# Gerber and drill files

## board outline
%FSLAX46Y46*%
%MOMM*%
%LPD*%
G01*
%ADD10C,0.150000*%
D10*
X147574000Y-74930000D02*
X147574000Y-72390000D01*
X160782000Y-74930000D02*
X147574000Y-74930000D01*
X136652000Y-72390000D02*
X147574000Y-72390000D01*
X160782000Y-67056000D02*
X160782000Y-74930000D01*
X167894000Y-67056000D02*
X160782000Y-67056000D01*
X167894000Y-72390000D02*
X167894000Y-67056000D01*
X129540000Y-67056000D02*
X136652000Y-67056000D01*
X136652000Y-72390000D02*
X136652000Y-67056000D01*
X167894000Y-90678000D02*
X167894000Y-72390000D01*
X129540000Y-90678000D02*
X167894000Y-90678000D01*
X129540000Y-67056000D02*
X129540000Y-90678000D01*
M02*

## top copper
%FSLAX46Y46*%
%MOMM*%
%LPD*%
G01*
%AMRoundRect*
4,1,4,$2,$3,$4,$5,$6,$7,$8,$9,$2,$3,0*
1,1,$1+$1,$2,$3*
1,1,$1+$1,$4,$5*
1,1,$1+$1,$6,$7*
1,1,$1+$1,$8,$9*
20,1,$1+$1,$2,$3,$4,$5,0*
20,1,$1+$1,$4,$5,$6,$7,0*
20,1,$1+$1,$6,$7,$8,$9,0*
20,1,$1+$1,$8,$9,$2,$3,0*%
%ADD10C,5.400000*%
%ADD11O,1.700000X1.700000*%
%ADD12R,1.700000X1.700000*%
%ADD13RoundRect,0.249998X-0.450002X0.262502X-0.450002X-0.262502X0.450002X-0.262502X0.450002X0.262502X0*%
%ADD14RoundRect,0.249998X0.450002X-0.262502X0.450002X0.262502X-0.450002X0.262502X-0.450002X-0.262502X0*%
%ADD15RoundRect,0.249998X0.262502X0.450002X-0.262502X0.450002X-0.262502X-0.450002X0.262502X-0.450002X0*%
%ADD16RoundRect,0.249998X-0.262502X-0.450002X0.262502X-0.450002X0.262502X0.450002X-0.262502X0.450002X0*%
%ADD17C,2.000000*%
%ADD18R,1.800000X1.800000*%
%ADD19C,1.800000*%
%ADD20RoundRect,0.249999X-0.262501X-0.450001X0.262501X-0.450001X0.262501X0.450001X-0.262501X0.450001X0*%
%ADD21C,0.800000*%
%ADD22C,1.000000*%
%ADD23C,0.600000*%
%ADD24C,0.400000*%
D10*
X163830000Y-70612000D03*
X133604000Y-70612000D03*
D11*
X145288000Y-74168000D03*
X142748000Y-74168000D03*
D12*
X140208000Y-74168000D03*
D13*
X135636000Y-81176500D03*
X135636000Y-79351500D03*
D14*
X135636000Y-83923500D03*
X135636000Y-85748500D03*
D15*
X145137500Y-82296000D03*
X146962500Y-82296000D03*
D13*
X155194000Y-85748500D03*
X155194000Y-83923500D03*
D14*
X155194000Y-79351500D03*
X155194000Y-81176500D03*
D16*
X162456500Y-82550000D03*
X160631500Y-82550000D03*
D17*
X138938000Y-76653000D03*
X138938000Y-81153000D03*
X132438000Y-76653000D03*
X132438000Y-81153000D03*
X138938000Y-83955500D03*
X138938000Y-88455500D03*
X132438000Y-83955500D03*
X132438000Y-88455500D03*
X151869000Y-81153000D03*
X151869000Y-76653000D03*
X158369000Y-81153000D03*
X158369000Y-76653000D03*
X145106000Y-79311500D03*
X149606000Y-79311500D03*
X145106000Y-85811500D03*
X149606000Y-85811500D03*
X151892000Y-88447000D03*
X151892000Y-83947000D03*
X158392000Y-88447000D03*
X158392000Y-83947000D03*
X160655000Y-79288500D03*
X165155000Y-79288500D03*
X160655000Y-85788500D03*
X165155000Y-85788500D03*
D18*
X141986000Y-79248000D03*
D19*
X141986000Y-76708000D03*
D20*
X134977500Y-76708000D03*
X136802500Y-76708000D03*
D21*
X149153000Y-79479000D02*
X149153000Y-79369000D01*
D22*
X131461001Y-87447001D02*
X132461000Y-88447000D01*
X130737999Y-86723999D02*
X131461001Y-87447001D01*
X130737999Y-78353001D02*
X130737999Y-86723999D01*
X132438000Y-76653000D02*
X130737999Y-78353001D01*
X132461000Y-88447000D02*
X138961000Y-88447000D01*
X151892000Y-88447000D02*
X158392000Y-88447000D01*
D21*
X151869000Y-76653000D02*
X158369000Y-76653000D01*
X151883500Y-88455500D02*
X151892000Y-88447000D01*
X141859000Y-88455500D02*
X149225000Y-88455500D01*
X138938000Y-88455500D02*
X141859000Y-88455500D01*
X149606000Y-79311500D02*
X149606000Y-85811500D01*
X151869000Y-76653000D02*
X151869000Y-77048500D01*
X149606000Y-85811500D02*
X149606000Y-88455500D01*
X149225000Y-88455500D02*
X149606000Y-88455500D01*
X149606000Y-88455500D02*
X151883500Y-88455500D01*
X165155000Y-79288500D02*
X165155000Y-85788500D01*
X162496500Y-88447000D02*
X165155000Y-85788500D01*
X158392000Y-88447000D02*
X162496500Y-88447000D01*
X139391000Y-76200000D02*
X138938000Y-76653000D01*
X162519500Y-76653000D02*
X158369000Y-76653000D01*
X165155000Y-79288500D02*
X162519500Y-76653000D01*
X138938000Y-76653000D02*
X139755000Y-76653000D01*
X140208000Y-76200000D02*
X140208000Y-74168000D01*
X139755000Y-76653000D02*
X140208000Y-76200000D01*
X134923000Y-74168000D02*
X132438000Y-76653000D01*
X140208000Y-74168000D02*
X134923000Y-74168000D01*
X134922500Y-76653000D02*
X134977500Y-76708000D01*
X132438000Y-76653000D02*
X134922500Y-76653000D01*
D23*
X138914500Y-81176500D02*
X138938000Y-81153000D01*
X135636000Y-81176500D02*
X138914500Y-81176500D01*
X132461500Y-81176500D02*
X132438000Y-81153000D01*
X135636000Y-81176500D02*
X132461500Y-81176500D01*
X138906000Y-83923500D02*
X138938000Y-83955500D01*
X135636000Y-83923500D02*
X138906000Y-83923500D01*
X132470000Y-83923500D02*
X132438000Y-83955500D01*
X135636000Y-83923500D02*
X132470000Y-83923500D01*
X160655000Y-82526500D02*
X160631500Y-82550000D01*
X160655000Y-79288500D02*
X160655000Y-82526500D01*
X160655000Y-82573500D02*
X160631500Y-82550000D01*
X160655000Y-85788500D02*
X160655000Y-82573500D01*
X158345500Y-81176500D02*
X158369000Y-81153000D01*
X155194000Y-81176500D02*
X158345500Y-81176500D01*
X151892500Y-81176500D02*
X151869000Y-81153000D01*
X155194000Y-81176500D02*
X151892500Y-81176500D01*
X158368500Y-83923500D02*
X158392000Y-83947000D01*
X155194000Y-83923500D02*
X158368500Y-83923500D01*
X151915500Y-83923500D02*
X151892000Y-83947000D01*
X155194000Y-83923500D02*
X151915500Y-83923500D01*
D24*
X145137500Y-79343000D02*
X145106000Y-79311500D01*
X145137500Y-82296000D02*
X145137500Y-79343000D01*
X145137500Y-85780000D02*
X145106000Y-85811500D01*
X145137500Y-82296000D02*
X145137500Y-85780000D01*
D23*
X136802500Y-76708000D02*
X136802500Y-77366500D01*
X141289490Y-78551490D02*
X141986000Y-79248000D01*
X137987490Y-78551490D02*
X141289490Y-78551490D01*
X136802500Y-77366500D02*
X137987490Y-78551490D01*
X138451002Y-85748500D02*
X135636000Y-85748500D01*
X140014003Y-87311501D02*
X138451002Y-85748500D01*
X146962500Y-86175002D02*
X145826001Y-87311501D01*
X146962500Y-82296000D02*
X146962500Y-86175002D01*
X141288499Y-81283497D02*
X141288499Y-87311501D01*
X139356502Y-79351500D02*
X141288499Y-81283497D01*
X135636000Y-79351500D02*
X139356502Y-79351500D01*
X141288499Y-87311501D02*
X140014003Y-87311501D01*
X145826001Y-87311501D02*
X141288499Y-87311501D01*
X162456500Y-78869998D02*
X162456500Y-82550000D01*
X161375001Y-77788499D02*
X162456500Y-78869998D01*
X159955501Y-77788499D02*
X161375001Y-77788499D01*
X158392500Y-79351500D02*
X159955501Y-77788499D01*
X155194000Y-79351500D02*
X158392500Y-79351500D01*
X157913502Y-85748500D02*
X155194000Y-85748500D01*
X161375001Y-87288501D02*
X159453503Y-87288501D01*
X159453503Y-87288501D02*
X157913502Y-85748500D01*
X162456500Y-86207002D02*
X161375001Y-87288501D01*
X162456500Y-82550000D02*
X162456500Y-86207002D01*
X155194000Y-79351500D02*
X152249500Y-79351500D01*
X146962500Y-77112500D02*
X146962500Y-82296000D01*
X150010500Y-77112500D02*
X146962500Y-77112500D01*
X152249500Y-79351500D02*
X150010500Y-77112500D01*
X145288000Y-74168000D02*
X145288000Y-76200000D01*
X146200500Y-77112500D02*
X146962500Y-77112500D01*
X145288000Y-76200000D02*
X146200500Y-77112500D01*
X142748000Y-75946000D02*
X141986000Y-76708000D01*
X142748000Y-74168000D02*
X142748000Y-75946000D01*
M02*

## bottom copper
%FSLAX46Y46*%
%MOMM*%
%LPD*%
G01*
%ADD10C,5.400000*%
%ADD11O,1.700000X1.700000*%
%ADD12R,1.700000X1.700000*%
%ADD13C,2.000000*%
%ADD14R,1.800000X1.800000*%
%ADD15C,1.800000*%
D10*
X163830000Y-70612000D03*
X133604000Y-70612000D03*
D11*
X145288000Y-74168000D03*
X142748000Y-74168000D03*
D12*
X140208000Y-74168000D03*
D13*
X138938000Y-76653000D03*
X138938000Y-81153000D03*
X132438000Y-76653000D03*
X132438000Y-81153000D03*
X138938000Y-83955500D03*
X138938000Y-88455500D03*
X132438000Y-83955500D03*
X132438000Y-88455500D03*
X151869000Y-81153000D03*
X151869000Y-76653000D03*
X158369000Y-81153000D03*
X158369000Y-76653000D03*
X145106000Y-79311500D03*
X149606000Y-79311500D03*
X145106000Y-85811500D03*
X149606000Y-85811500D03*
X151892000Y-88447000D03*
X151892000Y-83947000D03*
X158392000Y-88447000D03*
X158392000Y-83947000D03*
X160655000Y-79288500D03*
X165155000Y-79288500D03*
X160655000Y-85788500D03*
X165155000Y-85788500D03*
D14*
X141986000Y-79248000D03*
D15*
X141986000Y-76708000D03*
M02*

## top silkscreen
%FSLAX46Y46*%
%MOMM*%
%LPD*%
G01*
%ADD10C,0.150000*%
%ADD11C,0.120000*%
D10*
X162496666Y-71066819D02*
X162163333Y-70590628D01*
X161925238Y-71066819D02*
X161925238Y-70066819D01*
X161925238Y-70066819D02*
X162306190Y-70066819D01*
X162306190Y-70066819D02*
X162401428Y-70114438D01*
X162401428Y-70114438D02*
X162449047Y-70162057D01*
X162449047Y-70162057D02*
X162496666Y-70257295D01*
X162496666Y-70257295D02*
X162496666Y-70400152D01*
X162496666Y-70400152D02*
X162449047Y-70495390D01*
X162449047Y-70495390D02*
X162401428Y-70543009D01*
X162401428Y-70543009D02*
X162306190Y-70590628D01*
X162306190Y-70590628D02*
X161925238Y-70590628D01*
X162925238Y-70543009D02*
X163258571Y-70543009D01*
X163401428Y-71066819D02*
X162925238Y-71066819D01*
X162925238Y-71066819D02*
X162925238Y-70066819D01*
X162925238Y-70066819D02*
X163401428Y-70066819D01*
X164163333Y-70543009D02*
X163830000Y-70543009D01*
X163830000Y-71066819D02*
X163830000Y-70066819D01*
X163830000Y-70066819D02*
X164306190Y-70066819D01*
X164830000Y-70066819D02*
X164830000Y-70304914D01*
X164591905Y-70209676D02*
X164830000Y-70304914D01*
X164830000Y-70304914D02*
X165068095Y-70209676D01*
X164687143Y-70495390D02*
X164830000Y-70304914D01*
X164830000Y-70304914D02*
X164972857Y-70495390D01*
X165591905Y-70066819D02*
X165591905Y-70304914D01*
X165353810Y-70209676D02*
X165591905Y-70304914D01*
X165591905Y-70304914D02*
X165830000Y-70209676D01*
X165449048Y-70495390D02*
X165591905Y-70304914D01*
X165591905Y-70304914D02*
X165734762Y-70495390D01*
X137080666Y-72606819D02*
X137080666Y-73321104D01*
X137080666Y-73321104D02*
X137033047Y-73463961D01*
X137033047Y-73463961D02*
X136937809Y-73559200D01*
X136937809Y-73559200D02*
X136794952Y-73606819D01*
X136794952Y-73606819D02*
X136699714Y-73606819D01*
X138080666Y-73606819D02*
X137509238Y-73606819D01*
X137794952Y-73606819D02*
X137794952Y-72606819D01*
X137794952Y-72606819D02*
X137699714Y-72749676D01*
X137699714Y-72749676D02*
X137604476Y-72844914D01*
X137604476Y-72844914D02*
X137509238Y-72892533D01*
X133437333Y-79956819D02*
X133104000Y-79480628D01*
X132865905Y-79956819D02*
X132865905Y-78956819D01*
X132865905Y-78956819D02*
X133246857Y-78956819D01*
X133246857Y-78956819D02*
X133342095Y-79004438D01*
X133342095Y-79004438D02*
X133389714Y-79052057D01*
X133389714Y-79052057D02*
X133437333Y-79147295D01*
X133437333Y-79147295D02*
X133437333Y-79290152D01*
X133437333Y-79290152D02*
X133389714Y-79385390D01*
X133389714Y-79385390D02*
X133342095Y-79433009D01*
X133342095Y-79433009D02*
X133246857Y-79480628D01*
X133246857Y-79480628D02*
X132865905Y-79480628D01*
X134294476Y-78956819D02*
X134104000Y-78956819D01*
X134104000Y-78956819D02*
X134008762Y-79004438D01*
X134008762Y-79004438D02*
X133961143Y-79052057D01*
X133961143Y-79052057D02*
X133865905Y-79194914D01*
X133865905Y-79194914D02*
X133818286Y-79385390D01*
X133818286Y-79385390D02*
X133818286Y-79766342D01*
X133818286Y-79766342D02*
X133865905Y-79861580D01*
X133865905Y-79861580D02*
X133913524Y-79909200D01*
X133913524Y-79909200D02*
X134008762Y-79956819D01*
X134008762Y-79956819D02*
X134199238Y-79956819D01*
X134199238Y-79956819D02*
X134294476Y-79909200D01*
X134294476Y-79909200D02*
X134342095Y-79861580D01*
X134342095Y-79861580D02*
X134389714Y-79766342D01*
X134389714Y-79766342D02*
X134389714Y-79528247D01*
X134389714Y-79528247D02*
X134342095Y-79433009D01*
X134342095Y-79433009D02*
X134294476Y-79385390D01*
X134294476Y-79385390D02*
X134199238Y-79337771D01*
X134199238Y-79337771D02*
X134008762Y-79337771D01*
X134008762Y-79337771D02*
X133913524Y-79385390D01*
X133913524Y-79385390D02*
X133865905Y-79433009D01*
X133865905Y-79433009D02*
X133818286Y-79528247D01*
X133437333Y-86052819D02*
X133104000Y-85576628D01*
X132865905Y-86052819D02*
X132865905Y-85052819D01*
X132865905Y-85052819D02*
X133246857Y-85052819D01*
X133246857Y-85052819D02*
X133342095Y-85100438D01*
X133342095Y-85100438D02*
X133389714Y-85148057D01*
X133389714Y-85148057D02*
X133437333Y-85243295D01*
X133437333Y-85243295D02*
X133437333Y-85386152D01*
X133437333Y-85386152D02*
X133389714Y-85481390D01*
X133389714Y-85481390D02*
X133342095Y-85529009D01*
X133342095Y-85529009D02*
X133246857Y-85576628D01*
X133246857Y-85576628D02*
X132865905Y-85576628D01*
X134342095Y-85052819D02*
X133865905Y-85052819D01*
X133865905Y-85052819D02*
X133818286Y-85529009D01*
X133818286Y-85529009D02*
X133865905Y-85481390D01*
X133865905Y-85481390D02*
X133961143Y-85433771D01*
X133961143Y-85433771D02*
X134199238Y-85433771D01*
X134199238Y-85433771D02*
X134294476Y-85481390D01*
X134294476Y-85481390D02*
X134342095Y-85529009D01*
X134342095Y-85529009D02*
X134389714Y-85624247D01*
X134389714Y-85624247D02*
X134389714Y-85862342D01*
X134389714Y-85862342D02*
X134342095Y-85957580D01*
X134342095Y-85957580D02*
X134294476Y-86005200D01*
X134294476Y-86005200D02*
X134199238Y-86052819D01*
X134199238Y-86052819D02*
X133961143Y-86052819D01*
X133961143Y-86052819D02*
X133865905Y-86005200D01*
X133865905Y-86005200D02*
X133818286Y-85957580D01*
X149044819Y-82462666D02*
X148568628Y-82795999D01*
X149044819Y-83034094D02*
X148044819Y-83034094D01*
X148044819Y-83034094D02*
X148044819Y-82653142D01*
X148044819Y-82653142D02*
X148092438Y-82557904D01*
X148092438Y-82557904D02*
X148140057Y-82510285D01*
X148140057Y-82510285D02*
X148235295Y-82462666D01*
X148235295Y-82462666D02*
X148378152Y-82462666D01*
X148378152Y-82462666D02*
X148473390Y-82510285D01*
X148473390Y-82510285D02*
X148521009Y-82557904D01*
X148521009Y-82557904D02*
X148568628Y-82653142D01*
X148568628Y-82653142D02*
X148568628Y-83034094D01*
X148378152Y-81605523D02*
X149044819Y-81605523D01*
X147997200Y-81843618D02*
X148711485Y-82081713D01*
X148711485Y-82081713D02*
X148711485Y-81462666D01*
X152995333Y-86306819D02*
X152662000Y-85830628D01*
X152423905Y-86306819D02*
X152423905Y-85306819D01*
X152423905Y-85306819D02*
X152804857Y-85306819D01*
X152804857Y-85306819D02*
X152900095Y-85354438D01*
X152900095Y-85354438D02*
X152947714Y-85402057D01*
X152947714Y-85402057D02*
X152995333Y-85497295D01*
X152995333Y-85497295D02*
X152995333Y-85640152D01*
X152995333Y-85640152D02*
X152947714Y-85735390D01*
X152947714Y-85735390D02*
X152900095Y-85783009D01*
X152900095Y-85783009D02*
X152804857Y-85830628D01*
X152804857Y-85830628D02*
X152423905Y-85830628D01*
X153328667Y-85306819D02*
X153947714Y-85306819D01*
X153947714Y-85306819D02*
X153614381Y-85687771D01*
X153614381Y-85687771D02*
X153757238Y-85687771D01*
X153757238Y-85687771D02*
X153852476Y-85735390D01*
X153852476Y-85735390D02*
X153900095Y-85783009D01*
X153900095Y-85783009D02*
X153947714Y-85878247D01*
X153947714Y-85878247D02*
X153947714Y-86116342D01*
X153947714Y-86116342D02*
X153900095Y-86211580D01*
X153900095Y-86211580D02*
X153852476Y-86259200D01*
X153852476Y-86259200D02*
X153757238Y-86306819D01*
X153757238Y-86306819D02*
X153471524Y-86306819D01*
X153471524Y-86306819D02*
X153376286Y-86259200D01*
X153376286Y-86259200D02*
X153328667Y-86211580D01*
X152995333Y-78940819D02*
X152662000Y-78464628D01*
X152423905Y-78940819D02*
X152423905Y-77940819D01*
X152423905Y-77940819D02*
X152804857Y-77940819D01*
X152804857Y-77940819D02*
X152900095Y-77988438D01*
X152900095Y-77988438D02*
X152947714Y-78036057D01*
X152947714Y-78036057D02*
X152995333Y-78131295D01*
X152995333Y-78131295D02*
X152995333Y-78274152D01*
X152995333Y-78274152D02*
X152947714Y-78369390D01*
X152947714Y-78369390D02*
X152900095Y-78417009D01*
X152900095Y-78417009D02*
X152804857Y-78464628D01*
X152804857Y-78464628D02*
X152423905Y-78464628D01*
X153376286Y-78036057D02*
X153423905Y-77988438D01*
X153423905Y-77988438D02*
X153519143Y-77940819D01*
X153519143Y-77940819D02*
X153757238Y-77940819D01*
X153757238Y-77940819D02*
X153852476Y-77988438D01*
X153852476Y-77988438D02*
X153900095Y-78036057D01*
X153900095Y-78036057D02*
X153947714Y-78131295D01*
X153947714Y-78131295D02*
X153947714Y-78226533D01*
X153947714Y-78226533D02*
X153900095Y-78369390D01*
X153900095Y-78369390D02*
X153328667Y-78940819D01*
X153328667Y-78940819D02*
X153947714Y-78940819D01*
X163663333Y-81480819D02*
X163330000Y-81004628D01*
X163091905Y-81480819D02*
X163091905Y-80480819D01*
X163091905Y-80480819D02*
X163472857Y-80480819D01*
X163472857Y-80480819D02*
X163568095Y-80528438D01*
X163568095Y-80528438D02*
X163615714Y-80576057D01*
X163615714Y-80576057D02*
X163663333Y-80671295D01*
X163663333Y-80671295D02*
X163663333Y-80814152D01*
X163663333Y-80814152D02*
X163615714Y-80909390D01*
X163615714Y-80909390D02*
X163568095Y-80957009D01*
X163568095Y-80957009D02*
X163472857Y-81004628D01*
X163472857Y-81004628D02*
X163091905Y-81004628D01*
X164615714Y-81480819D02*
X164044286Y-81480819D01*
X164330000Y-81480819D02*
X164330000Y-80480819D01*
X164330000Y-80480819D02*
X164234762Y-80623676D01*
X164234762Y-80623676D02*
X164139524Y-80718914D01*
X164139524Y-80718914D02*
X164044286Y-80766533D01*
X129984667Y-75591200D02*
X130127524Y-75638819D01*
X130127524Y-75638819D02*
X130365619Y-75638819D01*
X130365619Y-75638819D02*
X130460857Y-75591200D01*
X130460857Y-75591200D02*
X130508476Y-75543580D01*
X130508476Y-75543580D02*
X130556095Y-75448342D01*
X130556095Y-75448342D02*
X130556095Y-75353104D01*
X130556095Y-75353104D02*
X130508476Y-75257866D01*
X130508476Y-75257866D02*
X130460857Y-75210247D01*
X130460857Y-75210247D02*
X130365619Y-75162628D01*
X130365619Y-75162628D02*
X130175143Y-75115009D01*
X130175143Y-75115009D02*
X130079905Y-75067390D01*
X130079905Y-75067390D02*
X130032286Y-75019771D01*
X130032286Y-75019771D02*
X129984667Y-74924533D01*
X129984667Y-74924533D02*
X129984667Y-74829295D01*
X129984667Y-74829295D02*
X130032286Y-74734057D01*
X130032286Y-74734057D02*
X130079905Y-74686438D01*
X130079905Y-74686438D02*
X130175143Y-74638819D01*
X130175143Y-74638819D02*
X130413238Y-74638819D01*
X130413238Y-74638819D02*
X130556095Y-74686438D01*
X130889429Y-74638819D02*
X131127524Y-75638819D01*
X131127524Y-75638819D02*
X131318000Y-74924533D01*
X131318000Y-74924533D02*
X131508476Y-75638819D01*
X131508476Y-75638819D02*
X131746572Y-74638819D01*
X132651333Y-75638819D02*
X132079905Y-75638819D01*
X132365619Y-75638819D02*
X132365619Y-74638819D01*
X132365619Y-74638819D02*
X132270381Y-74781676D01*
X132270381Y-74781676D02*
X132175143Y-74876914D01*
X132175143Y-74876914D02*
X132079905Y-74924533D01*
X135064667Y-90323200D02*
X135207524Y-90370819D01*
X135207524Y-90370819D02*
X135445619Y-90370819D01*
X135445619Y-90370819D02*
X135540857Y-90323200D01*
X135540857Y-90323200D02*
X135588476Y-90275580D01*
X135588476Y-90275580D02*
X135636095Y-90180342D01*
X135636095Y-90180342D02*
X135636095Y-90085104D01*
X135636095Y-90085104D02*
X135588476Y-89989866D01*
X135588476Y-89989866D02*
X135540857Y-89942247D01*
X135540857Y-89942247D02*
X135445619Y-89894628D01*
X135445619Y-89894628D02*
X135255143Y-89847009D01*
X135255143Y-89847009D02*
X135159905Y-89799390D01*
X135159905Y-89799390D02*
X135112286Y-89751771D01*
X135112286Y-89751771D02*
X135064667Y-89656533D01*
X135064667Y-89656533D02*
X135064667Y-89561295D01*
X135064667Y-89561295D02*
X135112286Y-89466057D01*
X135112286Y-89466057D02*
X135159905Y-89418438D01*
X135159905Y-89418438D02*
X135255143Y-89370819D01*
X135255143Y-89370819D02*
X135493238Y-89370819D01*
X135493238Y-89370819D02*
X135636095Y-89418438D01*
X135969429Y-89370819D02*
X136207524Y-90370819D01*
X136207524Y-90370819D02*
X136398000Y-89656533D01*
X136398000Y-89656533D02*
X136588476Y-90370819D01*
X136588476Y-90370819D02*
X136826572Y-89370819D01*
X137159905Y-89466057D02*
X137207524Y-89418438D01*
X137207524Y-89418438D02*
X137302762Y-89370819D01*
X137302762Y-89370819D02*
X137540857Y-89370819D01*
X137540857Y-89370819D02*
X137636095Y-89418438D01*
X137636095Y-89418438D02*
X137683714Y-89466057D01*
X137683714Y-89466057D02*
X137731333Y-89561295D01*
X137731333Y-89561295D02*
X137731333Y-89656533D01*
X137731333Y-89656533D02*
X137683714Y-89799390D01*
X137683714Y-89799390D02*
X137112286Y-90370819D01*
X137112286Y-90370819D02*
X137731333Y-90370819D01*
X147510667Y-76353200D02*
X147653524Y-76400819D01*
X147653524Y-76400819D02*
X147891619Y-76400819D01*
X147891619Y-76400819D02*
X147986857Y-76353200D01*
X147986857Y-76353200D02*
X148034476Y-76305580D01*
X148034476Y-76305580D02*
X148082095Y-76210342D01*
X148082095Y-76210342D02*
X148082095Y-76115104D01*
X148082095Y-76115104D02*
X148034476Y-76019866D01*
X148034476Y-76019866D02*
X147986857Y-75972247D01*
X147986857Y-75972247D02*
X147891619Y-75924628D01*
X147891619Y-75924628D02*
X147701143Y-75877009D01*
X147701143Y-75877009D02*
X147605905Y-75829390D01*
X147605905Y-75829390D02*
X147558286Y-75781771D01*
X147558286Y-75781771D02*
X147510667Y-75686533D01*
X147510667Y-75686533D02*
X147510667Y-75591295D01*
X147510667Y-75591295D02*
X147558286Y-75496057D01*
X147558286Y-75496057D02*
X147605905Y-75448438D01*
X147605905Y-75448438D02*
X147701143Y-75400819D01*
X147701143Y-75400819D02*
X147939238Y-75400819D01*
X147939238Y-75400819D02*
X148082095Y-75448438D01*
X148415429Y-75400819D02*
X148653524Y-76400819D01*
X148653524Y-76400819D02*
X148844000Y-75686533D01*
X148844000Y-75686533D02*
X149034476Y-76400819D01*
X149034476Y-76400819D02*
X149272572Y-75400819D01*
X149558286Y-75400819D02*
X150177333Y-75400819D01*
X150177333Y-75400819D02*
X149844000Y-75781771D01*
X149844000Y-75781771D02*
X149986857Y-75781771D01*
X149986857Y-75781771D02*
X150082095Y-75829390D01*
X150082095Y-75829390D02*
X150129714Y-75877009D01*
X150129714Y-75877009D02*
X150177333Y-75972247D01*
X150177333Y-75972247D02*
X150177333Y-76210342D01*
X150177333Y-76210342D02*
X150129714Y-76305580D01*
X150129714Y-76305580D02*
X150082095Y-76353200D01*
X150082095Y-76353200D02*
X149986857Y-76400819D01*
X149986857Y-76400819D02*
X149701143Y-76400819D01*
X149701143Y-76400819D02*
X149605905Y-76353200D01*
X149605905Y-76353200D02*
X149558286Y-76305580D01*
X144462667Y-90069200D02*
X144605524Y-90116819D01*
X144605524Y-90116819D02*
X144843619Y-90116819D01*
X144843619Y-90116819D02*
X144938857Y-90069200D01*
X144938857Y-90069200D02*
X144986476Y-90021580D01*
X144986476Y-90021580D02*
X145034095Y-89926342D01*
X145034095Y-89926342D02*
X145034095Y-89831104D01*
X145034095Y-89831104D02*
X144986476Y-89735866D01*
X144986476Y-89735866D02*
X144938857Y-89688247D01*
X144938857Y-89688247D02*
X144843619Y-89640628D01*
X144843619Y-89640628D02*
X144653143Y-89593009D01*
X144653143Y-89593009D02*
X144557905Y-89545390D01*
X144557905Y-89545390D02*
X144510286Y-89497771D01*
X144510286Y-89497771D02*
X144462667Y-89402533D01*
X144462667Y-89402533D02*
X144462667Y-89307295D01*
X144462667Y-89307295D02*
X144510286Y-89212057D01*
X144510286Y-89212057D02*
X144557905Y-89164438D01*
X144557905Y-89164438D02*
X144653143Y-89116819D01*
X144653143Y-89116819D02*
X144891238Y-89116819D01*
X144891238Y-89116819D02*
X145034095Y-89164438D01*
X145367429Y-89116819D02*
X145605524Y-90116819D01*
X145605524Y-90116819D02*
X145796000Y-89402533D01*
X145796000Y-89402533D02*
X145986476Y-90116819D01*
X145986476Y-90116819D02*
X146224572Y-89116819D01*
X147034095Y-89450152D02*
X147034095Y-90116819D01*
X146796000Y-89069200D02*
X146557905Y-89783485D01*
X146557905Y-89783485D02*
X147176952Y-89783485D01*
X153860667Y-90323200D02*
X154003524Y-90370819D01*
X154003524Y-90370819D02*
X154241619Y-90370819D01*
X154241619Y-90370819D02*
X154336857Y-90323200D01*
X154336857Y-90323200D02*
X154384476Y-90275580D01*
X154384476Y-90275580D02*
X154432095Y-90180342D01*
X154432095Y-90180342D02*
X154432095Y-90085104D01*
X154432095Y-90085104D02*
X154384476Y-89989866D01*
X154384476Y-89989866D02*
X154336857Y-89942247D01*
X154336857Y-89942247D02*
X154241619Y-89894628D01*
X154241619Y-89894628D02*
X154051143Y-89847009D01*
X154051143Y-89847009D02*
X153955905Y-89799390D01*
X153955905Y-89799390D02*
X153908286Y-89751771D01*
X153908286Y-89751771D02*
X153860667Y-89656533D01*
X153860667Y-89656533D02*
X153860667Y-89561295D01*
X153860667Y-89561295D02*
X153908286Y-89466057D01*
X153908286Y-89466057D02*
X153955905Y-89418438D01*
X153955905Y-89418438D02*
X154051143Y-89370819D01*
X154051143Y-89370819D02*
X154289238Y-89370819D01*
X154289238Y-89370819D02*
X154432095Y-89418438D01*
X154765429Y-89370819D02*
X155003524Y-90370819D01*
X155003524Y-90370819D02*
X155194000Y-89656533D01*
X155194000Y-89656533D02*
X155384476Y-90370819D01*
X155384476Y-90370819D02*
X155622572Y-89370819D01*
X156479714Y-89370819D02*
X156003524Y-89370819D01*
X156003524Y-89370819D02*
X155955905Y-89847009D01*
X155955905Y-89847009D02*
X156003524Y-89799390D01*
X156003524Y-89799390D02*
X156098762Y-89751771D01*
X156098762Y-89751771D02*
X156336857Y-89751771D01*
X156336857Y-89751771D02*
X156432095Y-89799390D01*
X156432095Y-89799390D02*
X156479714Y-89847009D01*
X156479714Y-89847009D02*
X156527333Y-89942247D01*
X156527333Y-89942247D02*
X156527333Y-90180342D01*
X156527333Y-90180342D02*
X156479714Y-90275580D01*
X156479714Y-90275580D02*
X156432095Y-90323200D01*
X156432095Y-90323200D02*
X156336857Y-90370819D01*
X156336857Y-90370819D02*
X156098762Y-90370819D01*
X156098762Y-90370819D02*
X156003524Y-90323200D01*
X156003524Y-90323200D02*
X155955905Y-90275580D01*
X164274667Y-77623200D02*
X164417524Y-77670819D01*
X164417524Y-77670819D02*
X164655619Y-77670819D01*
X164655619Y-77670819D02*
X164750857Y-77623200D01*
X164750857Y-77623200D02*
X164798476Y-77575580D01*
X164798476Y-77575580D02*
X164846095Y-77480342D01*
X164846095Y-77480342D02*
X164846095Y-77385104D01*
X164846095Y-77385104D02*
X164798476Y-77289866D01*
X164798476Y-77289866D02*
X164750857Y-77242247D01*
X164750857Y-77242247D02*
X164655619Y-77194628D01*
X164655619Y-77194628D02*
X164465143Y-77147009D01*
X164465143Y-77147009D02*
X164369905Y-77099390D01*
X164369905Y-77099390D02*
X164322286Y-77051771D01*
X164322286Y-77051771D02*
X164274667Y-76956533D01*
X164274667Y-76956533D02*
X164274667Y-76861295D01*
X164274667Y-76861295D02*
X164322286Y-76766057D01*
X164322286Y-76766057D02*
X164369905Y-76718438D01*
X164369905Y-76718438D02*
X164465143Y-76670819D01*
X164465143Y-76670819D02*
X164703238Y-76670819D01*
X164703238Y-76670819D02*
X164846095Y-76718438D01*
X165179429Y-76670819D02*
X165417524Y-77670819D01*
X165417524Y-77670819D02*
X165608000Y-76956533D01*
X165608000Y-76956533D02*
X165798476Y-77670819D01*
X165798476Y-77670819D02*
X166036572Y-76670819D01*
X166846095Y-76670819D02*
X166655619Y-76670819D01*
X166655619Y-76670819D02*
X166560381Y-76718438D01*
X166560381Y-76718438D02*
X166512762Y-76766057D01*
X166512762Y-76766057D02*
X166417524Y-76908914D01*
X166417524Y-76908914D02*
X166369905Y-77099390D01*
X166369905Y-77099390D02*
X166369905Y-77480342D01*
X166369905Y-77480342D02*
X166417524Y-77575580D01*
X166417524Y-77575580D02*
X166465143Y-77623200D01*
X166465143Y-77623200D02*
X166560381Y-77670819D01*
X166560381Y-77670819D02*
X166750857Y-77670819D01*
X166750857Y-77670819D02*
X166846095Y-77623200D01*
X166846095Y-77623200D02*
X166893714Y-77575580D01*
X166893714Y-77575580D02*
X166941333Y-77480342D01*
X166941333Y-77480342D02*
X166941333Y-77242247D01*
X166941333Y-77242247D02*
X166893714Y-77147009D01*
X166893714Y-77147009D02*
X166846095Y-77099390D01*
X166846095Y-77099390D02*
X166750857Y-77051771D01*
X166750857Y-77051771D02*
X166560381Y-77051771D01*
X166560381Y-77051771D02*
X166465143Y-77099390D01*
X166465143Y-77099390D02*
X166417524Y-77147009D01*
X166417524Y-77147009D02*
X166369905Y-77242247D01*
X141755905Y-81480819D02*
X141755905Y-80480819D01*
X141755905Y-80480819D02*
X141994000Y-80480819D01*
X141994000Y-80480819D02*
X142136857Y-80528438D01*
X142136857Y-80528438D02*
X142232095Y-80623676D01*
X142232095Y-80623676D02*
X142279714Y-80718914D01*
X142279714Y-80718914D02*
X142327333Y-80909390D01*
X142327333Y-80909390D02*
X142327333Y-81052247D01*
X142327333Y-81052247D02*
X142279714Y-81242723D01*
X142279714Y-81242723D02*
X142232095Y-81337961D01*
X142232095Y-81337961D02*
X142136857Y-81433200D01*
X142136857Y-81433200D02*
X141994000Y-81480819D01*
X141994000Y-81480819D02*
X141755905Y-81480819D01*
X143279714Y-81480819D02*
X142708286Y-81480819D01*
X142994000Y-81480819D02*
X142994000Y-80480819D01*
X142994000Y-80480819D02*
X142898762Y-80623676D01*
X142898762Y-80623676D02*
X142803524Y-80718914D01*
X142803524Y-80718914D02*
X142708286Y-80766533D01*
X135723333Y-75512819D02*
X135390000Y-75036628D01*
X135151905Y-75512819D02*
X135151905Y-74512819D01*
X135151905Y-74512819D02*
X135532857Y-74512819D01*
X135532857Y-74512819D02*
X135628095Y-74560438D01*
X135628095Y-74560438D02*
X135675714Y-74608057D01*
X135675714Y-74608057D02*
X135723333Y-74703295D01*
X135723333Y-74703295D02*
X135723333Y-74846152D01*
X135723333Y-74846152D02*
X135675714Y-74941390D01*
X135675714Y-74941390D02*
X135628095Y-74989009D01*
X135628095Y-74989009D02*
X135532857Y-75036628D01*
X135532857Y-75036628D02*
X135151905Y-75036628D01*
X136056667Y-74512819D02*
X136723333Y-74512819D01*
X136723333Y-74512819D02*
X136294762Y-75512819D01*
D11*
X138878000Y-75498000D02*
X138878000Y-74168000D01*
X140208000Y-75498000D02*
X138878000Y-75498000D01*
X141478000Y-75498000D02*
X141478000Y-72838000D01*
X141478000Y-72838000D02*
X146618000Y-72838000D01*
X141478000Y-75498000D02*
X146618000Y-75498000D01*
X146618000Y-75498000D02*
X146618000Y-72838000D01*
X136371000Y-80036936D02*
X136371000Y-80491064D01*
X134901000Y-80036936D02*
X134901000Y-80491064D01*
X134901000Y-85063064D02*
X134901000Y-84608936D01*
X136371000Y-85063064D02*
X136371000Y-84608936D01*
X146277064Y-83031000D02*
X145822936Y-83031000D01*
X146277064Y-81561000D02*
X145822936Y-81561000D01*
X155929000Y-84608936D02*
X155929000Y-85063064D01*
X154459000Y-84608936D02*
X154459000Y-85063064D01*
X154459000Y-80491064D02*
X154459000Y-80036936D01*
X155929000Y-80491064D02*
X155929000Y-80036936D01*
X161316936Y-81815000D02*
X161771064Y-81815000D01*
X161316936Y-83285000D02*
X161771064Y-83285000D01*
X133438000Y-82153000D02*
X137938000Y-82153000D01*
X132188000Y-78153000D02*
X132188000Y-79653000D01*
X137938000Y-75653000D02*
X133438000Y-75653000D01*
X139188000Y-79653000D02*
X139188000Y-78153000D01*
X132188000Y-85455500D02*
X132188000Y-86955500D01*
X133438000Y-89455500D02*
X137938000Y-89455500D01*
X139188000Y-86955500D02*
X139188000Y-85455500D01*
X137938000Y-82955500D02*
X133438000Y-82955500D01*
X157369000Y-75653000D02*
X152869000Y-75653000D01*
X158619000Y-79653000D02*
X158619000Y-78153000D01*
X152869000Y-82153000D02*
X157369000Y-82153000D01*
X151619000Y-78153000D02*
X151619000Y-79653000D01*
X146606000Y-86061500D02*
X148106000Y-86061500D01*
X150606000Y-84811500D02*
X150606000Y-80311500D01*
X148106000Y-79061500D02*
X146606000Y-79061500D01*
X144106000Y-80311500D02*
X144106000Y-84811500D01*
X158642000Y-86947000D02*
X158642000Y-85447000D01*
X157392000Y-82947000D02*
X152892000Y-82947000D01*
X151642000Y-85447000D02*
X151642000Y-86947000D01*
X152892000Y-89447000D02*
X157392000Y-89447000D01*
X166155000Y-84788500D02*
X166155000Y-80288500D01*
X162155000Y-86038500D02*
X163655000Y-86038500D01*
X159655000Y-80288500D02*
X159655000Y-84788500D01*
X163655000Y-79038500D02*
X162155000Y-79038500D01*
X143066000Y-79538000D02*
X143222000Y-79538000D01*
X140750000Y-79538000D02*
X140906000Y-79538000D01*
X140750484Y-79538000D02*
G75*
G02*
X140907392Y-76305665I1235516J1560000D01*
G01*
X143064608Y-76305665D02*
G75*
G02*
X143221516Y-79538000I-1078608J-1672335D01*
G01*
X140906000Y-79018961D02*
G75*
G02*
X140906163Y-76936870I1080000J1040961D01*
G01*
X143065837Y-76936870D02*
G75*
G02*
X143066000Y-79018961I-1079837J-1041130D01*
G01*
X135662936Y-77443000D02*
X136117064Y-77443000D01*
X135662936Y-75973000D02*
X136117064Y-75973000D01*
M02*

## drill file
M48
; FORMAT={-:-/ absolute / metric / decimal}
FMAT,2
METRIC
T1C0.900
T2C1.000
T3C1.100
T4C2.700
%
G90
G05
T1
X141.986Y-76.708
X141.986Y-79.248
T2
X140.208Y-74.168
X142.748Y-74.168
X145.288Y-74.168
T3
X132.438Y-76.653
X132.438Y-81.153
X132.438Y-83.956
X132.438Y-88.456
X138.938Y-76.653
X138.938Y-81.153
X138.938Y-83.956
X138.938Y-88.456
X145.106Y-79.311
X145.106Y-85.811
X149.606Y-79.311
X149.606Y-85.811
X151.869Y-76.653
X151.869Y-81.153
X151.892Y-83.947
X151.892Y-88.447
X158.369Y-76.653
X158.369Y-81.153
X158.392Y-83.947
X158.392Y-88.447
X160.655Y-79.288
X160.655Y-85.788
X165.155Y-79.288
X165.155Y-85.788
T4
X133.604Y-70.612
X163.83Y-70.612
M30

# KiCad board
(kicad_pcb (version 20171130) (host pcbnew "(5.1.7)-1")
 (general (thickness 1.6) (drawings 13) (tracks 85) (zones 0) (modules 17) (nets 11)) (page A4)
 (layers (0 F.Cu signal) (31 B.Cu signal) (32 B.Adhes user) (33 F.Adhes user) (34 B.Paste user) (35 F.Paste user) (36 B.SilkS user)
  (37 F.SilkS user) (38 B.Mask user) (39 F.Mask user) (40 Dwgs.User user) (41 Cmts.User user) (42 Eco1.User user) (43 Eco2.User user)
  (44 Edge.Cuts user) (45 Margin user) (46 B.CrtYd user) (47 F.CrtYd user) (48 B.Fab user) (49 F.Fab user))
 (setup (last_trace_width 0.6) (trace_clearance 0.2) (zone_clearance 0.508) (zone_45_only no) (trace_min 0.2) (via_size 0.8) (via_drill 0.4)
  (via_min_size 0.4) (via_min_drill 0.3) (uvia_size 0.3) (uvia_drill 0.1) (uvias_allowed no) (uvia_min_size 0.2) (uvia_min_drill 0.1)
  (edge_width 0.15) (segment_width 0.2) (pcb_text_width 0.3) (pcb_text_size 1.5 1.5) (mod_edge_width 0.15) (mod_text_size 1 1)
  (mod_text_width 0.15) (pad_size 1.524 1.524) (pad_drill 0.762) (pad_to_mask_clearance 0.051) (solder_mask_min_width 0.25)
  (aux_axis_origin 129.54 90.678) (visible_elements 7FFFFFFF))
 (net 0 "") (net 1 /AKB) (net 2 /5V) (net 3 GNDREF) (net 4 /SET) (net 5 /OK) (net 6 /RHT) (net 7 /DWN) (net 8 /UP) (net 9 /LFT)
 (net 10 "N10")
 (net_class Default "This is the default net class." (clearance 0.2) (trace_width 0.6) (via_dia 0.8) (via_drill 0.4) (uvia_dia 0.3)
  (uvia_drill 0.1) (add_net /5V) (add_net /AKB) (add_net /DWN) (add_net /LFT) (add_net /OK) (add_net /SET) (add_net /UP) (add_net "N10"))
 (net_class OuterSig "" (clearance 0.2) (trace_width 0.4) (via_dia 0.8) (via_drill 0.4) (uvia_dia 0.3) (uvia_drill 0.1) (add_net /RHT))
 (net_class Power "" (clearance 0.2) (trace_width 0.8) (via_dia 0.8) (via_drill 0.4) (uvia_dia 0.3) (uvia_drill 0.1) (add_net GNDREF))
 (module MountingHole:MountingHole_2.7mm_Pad (layer F.Cu) (at 163.83 70.612)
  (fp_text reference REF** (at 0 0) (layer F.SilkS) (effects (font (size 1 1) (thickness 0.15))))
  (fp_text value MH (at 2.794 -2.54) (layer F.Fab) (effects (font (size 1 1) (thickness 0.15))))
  (pad 1 thru_hole circle (at 0 0) (size 5.4 5.4) (drill 2.7) (layers *.Cu *.Mask)))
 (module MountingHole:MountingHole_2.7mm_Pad (layer F.Cu) (at 133.604 70.612)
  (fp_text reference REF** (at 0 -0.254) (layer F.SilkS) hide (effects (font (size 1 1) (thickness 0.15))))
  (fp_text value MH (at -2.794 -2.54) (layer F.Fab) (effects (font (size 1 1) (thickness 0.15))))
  (pad 1 thru_hole circle (at 0 0) (size 5.4 5.4) (drill 2.7) (layers *.Cu *.Mask)))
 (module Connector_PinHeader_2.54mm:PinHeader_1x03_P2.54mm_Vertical (layer F.Cu) (at 140.208 74.168 90)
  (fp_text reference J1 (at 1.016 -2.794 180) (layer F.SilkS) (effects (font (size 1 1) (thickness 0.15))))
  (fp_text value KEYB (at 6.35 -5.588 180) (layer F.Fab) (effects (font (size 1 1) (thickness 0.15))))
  (fp_line (start -1.33 -1.33) (end 0 -1.33) (layer F.SilkS) (width 0.12))
  (fp_line (start -1.33 0) (end -1.33 -1.33) (layer F.SilkS) (width 0.12))
  (fp_line (start -1.33 1.27) (end 1.33 1.27) (layer F.SilkS) (width 0.12))
  (fp_line (start 1.33 1.27) (end 1.33 6.41) (layer F.SilkS) (width 0.12))
  (fp_line (start -1.33 1.27) (end -1.33 6.41) (layer F.SilkS) (width 0.12))
  (fp_line (start -1.33 6.41) (end 1.33 6.41) (layer F.SilkS) (width 0.12))
  (pad 3 thru_hole oval (at 0 5.08 90) (size 1.7 1.7) (drill 1) (layers *.Cu *.Mask) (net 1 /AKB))
  (pad 2 thru_hole oval (at 0 2.54 90) (size 1.7 1.7) (drill 1) (layers *.Cu *.Mask) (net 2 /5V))
  (pad 1 thru_hole rect (at 0 0 90) (size 1.7 1.7) (drill 1) (layers *.Cu *.Mask) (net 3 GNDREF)))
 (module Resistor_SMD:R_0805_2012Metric (layer F.Cu) (at 135.636 80.264 270)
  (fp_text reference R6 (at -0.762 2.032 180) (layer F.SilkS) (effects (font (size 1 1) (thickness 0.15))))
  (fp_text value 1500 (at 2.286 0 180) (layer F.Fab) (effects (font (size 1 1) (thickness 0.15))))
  (fp_line (start -0.227064 -0.735) (end 0.227064 -0.735) (layer F.SilkS) (width 0.12))
  (fp_line (start -0.227064 0.735) (end 0.227064 0.735) (layer F.SilkS) (width 0.12))
  (pad 2 smd roundrect (at 0.9125 0 270) (size 1.025 1.4) (layers F.Cu F.Paste F.Mask) (roundrect_rratio 0.2439004878048781) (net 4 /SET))
  (pad 1 smd roundrect (at -0.9125 0 270) (size 1.025 1.4) (layers F.Cu F.Paste F.Mask) (roundrect_rratio 0.2439004878048781) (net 1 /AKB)))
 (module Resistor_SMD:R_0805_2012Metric (layer F.Cu) (at 135.636 84.836 90)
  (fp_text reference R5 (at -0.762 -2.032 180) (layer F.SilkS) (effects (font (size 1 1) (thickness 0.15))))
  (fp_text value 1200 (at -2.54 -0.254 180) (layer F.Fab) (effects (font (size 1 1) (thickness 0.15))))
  (fp_line (start -0.227064 -0.735) (end 0.227064 -0.735) (layer F.SilkS) (width 0.12))
  (fp_line (start -0.227064 0.735) (end 0.227064 0.735) (layer F.SilkS) (width 0.12))
  (pad 2 smd roundrect (at 0.9125 0 90) (size 1.025 1.4) (layers F.Cu F.Paste F.Mask) (roundrect_rratio 0.2439004878048781) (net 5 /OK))
  (pad 1 smd roundrect (at -0.9125 0 90) (size 1.025 1.4) (layers F.Cu F.Paste F.Mask) (roundrect_rratio 0.2439004878048781) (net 1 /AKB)))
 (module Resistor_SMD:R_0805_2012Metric (layer F.Cu) (at 146.05 82.296 180)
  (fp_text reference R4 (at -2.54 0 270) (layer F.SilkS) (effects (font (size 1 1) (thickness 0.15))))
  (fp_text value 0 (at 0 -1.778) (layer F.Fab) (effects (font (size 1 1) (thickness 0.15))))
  (fp_line (start -0.227064 -0.735) (end 0.227064 -0.735) (layer F.SilkS) (width 0.12))
  (fp_line (start -0.227064 0.735) (end 0.227064 0.735) (layer F.SilkS) (width 0.12))
  (pad 2 smd roundrect (at 0.9125 0 180) (size 1.025 1.4) (layers F.Cu F.Paste F.Mask) (roundrect_rratio 0.2439004878048781) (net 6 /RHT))
  (pad 1 smd roundrect (at -0.9125 0 180) (size 1.025 1.4) (layers F.Cu F.Paste F.Mask) (roundrect_rratio 0.2439004878048781) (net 1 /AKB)))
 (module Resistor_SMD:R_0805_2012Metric (layer F.Cu) (at 155.194 84.836 270)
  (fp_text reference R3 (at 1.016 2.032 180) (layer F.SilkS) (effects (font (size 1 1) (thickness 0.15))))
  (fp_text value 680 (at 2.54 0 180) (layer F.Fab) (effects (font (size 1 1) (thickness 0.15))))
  (fp_line (start -0.227064 -0.735) (end 0.227064 -0.735) (layer F.SilkS) (width 0.12))
  (fp_line (start -0.227064 0.735) (end 0.227064 0.735) (layer F.SilkS) (width 0.12))
  (pad 2 smd roundrect (at 0.9125 0 270) (size 1.025 1.4) (layers F.Cu F.Paste F.Mask) (roundrect_rratio 0.2439004878048781) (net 1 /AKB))
  (pad 1 smd roundrect (at -0.9125 0 270) (size 1.025 1.4) (layers F.Cu F.Paste F.Mask) (roundrect_rratio 0.2439004878048781) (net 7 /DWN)))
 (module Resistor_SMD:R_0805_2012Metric (layer F.Cu) (at 155.194 80.264 90)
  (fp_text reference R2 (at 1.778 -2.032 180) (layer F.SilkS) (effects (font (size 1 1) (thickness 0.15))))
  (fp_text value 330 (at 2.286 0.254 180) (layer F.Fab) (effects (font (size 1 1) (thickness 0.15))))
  (fp_line (start -0.227064 -0.735) (end 0.227064 -0.735) (layer F.SilkS) (width 0.12))
  (fp_line (start -0.227064 0.735) (end 0.227064 0.735) (layer F.SilkS) (width 0.12))
  (pad 2 smd roundrect (at 0.9125 0 90) (size 1.025 1.4) (layers F.Cu F.Paste F.Mask) (roundrect_rratio 0.2439004878048781) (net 1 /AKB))
  (pad 1 smd roundrect (at -0.9125 0 90) (size 1.025 1.4) (layers F.Cu F.Paste F.Mask) (roundrect_rratio 0.2439004878048781) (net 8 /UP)))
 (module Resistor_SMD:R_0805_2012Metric (layer F.Cu) (at 161.544 82.55)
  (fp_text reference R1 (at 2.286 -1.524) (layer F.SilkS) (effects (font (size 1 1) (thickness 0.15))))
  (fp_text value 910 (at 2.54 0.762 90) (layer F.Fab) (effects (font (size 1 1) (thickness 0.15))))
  (fp_line (start -0.227064 -0.735) (end 0.227064 -0.735) (layer F.SilkS) (width 0.12))
  (fp_line (start -0.227064 0.735) (end 0.227064 0.735) (layer F.SilkS) (width 0.12))
  (pad 2 smd roundrect (at 0.9125 0) (size 1.025 1.4) (layers F.Cu F.Paste F.Mask) (roundrect_rratio 0.2439004878048781) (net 1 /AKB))
  (pad 1 smd roundrect (at -0.9125 0) (size 1.025 1.4) (layers F.Cu F.Paste F.Mask) (roundrect_rratio 0.2439004878048781) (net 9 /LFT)))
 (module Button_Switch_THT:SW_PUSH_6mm (layer F.Cu) (at 132.438 76.653)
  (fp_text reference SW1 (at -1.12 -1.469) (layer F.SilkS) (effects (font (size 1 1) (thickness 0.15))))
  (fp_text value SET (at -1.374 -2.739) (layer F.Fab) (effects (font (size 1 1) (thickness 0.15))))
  (fp_line (start 1 5.5) (end 5.5 5.5) (layer F.SilkS) (width 0.12))
  (fp_line (start -0.25 1.5) (end -0.25 3) (layer F.SilkS) (width 0.12))
  (fp_line (start 5.5 -1) (end 1 -1) (layer F.SilkS) (width 0.12))
  (fp_line (start 6.75 3) (end 6.75 1.5) (layer F.SilkS) (width 0.12))
  (pad 1 thru_hole circle (at 6.5 0 90) (size 2 2) (drill 1.1) (layers *.Cu *.Mask) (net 3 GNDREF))
  (pad 2 thru_hole circle (at 6.5 4.5 90) (size 2 2) (drill 1.1) (layers *.Cu *.Mask) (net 4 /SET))
  (pad 1 thru_hole circle (at 0 0 90) (size 2 2) (drill 1.1) (layers *.Cu *.Mask) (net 3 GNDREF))
  (pad 2 thru_hole circle (at 0 4.5 90) (size 2 2) (drill 1.1) (layers *.Cu *.Mask) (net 4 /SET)))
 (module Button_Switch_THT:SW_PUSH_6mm (layer F.Cu) (at 138.938 88.4555 180)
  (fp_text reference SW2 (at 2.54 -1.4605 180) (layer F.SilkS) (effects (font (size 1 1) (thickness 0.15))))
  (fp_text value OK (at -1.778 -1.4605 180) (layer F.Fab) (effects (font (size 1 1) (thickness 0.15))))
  (fp_line (start 6.75 3) (end 6.75 1.5) (layer F.SilkS) (width 0.12))
  (fp_line (start 5.5 -1) (end 1 -1) (layer F.SilkS) (width 0.12))
  (fp_line (start -0.25 1.5) (end -0.25 3) (layer F.SilkS) (width 0.12))
  (fp_line (start 1 5.5) (end 5.5 5.5) (layer F.SilkS) (width 0.12))
  (pad 2 thru_hole circle (at 0 4.5 270) (size 2 2) (drill 1.1) (layers *.Cu *.Mask) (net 5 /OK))
  (pad 1 thru_hole circle (at 0 0 270) (size 2 2) (drill 1.1) (layers *.Cu *.Mask) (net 3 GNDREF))
  (pad 2 thru_hole circle (at 6.5 4.5 270) (size 2 2) (drill 1.1) (layers *.Cu *.Mask) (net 5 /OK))
  (pad 1 thru_hole circle (at 6.5 0 270) (size 2 2) (drill 1.1) (layers *.Cu *.Mask) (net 3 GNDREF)))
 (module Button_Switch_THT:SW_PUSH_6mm (layer F.Cu) (at 158.369 81.153 180)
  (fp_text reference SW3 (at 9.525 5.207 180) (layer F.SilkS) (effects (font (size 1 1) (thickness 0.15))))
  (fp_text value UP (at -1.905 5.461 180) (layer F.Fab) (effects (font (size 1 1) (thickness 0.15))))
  (fp_line (start 1 5.5) (end 5.5 5.5) (layer F.SilkS) (width 0.12))
  (fp_line (start -0.25 1.5) (end -0.25 3) (layer F.SilkS) (width 0.12))
  (fp_line (start 5.5 -1) (end 1 -1) (layer F.SilkS) (width 0.12))
  (fp_line (start 6.75 3) (end 6.75 1.5) (layer F.SilkS) (width 0.12))
  (pad 1 thru_hole circle (at 6.5 0 270) (size 2 2) (drill 1.1) (layers *.Cu *.Mask) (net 8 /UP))
  (pad 2 thru_hole circle (at 6.5 4.5 270) (size 2 2) (drill 1.1) (layers *.Cu *.Mask) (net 3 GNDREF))
  (pad 1 thru_hole circle (at 0 0 270) (size 2 2) (drill 1.1) (layers *.Cu *.Mask) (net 8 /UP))
  (pad 2 thru_hole circle (at 0 4.5 270) (size 2 2) (drill 1.1) (layers *.Cu *.Mask) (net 3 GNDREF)))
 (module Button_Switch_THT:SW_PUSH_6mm (layer F.Cu) (at 149.606 79.3115 270)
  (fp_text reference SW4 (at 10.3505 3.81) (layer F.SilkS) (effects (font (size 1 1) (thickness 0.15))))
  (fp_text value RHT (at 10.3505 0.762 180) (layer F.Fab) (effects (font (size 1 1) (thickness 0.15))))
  (fp_line (start 6.75 3) (end 6.75 1.5) (layer F.SilkS) (width 0.12))
  (fp_line (start 5.5 -1) (end 1 -1) (layer F.SilkS) (width 0.12))
  (fp_line (start -0.25 1.5) (end -0.25 3) (layer F.SilkS) (width 0.12))
  (fp_line (start 1 5.5) (end 5.5 5.5) (layer F.SilkS) (width 0.12))
  (pad 2 thru_hole circle (at 0 4.5) (size 2 2) (drill 1.1) (layers *.Cu *.Mask) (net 6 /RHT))
  (pad 1 thru_hole circle (at 0 0) (size 2 2) (drill 1.1) (layers *.Cu *.Mask) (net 3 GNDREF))
  (pad 2 thru_hole circle (at 6.5 4.5) (size 2 2) (drill 1.1) (layers *.Cu *.Mask) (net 6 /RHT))
  (pad 1 thru_hole circle (at 6.5 0) (size 2 2) (drill 1.1) (layers *.Cu *.Mask) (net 3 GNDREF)))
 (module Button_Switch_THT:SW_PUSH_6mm (layer F.Cu) (at 151.892 83.947)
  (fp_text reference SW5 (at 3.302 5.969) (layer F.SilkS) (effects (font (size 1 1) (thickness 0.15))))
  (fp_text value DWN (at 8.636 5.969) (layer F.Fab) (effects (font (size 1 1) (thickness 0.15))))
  (fp_line (start 6.75 3) (end 6.75 1.5) (layer F.SilkS) (width 0.12))
  (fp_line (start 5.5 -1) (end 1 -1) (layer F.SilkS) (width 0.12))
  (fp_line (start -0.25 1.5) (end -0.25 3) (layer F.SilkS) (width 0.12))
  (fp_line (start 1 5.5) (end 5.5 5.5) (layer F.SilkS) (width 0.12))
  (pad 2 thru_hole circle (at 0 4.5 90) (size 2 2) (drill 1.1) (layers *.Cu *.Mask) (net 3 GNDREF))
  (pad 1 thru_hole circle (at 0 0 90) (size 2 2) (drill 1.1) (layers *.Cu *.Mask) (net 7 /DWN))
  (pad 2 thru_hole circle (at 6.5 4.5 90) (size 2 2) (drill 1.1) (layers *.Cu *.Mask) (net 3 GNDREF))
  (pad 1 thru_hole circle (at 6.5 0 90) (size 2 2) (drill 1.1) (layers *.Cu *.Mask) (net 7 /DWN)))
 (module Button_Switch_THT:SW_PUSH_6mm (layer F.Cu) (at 160.655 85.7885 90)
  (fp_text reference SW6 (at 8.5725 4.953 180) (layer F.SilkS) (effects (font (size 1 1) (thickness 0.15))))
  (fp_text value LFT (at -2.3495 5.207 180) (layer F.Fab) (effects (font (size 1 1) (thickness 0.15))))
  (fp_line (start 1 5.5) (end 5.5 5.5) (layer F.SilkS) (width 0.12))
  (fp_line (start -0.25 1.5) (end -0.25 3) (layer F.SilkS) (width 0.12))
  (fp_line (start 5.5 -1) (end 1 -1) (layer F.SilkS) (width 0.12))
  (fp_line (start 6.75 3) (end 6.75 1.5) (layer F.SilkS) (width 0.12))
  (pad 1 thru_hole circle (at 6.5 0 180) (size 2 2) (drill 1.1) (layers *.Cu *.Mask) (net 9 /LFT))
  (pad 2 thru_hole circle (at 6.5 4.5 180) (size 2 2) (drill 1.1) (layers *.Cu *.Mask) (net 3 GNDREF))
  (pad 1 thru_hole circle (at 0 0 180) (size 2 2) (drill 1.1) (layers *.Cu *.Mask) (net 9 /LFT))
  (pad 2 thru_hole circle (at 0 4.5 180) (size 2 2) (drill 1.1) (layers *.Cu *.Mask) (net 3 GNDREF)))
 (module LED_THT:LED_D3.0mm (layer F.Cu) (at 141.986 79.248 90)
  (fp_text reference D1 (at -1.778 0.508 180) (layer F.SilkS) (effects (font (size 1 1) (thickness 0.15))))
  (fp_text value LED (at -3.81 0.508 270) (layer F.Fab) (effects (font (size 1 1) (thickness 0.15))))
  (fp_line (start -0.29 1.08) (end -0.29 1.236) (layer F.SilkS) (width 0.12))
  (fp_line (start -0.29 -1.236) (end -0.29 -1.08) (layer F.SilkS) (width 0.12))
  (fp_arc (start 1.27 0) (end -0.29 -1.235516) (angle 108.8) (layer F.SilkS) (width 0.12))
  (fp_arc (start 1.27 0) (end -0.29 1.235516) (angle -108.8) (layer F.SilkS) (width 0.12))
  (fp_arc (start 1.27 0) (end 0.229039 -1.08) (angle 87.9) (layer F.SilkS) (width 0.12))
  (fp_arc (start 1.27 0) (end 0.229039 1.08) (angle -87.9) (layer F.SilkS) (width 0.12))
  (pad 1 thru_hole rect (at 0 0 90) (size 1.8 1.8) (drill 0.9) (layers *.Cu *.Mask) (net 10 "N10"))
  (pad 2 thru_hole circle (at 2.54 0 90) (size 1.8 1.8) (drill 0.9) (layers *.Cu *.Mask) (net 2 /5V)))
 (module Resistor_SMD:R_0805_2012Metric (layer F.Cu) (at 135.89 76.708)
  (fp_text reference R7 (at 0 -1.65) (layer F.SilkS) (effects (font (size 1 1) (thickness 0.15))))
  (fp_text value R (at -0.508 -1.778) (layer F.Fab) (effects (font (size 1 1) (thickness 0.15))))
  (fp_line (start -0.227064 0.735) (end 0.227064 0.735) (layer F.SilkS) (width 0.12))
  (fp_line (start -0.227064 -0.735) (end 0.227064 -0.735) (layer F.SilkS) (width 0.12))
  (pad 1 smd roundrect (at -0.9125 0) (size 1.025 1.4) (layers F.Cu F.Paste F.Mask) (roundrect_rratio 0.2439014634146341) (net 3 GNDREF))
  (pad 2 smd roundrect (at 0.9125 0) (size 1.025 1.4) (layers F.Cu F.Paste F.Mask) (roundrect_rratio 0.2439014634146341) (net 10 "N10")))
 (gr_line (start 147.574 74.93) (end 147.574 72.39) (layer Edge.Cuts) (width 0.15))
 (gr_line (start 160.782 74.93) (end 147.574 74.93) (layer Edge.Cuts) (width 0.15))
 (gr_line (start 136.652 72.39) (end 147.574 72.39) (layer Edge.Cuts) (width 0.15))
 (gr_line (start 160.782 67.056) (end 160.782 74.93) (layer Edge.Cuts) (width 0.15))
 (gr_line (start 167.894 67.056) (end 160.782 67.056) (layer Edge.Cuts) (width 0.15))
 (gr_line (start 167.894 72.39) (end 167.894 67.056) (layer Edge.Cuts) (width 0.15))
 (gr_line (start 129.54 67.056) (end 136.652 67.056) (layer Edge.Cuts) (width 0.15))
 (gr_line (start 136.652 72.39) (end 136.652 67.056) (layer Edge.Cuts) (width 0.15))
 (gr_line (start 167.894 90.678) (end 167.894 72.39) (layer Edge.Cuts) (width 0.15))
 (gr_line (start 129.54 90.678) (end 167.894 90.678) (layer Edge.Cuts) (width 0.15))
 (gr_line (start 129.54 67.056) (end 129.54 90.678) (layer Edge.Cuts) (width 0.15))
 (segment (start 149.153 79.479) (end 149.153 79.369) (width 0.8) (layer F.Cu) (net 3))
 (segment (start 131.461001 87.447001) (end 132.461 88.447) (width 1) (layer F.Cu) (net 3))
 (segment (start 130.737999 86.723999) (end 131.461001 87.447001) (width 1) (layer F.Cu) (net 3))
 (segment (start 130.737999 78.353001) (end 130.737999 86.723999) (width 1) (layer F.Cu) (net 3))
 (segment (start 132.438 76.653) (end 130.737999 78.353001) (width 1) (layer F.Cu) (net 3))
 (segment (start 132.461 88.447) (end 138.961 88.447) (width 1) (layer F.Cu) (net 3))
 (segment (start 151.892 88.447) (end 158.392 88.447) (width 1) (layer F.Cu) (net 3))
 (segment (start 151.869 76.653) (end 158.369 76.653) (width 0.8) (layer F.Cu) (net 3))
 (segment (start 151.8835 88.4555) (end 151.892 88.447) (width 0.8) (layer F.Cu) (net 3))
 (segment (start 141.859 88.4555) (end 149.225 88.4555) (width 0.8) (layer F.Cu) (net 3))
 (segment (start 138.938 88.4555) (end 141.859 88.4555) (width 0.8) (layer F.Cu) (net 3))
 (segment (start 149.606 79.3115) (end 149.606 85.8115) (width 0.8) (layer F.Cu) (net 3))
 (segment (start 151.869 76.653) (end 151.869 77.0485) (width 0.8) (layer F.Cu) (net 3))
 (segment (start 149.606 85.8115) (end 149.606 88.4555) (width 0.8) (layer F.Cu) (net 3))
 (segment (start 149.225 88.4555) (end 149.606 88.4555) (width 0.8) (layer F.Cu) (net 3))
 (segment (start 149.606 88.4555) (end 151.8835 88.4555) (width 0.8) (layer F.Cu) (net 3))
 (segment (start 165.155 79.2885) (end 165.155 85.7885) (width 0.8) (layer F.Cu) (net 3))
 (segment (start 162.4965 88.447) (end 165.155 85.7885) (width 0.8) (layer F.Cu) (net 3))
 (segment (start 158.392 88.447) (end 162.4965 88.447) (width 0.8) (layer F.Cu) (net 3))
 (segment (start 139.391 76.2) (end 138.938 76.653) (width 0.8) (layer F.Cu) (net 3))
 (segment (start 162.5195 76.653) (end 158.369 76.653) (width 0.8) (layer F.Cu) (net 3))
 (segment (start 165.155 79.2885) (end 162.5195 76.653) (width 0.8) (layer F.Cu) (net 3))
 (segment (start 138.938 76.653) (end 139.755 76.653) (width 0.8) (layer F.Cu) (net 3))
 (segment (start 140.208 76.2) (end 140.208 74.168) (width 0.8) (layer F.Cu) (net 3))
 (segment (start 139.755 76.653) (end 140.208 76.2) (width 0.8) (layer F.Cu) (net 3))
 (segment (start 134.923 74.168) (end 132.438 76.653) (width 0.8) (layer F.Cu) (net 3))
 (segment (start 140.208 74.168) (end 134.923 74.168) (width 0.8) (layer F.Cu) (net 3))
 (segment (start 134.9225 76.653) (end 134.9775 76.708) (width 0.8) (layer F.Cu) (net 3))
 (segment (start 132.438 76.653) (end 134.9225 76.653) (width 0.8) (layer F.Cu) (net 3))
 (segment (start 138.9145 81.1765) (end 138.938 81.153) (width 0.6) (layer F.Cu) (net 4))
 (segment (start 135.636 81.1765) (end 138.9145 81.1765) (width 0.6) (layer F.Cu) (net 4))
 (segment (start 132.4615 81.1765) (end 132.438 81.153) (width 0.6) (layer F.Cu) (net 4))
 (segment (start 135.636 81.1765) (end 132.4615 81.1765) (width 0.6) (layer F.Cu) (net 4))
 (segment (start 138.906 83.9235) (end 138.938 83.9555) (width 0.6) (layer F.Cu) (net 5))
 (segment (start 135.636 83.9235) (end 138.906 83.9235) (width 0.6) (layer F.Cu) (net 5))
 (segment (start 132.47 83.9235) (end 132.438 83.9555) (width 0.6) (layer F.Cu) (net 5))
 (segment (start 135.636 83.9235) (end 132.47 83.9235) (width 0.6) (layer F.Cu) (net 5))
 (segment (start 160.655 82.5265) (end 160.6315 82.55) (width 0.6) (layer F.Cu) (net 9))
 (segment (start 160.655 79.2885) (end 160.655 82.5265) (width 0.6) (layer F.Cu) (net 9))
 (segment (start 160.655 82.5735) (end 160.6315 82.55) (width 0.6) (layer F.Cu) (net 9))
 (segment (start 160.655 85.7885) (end 160.655 82.5735) (width 0.6) (layer F.Cu) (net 9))
 (segment (start 158.3455 81.1765) (end 158.369 81.153) (width 0.6) (layer F.Cu) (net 8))
 (segment (start 155.194 81.1765) (end 158.3455 81.1765) (width 0.6) (layer F.Cu) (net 8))
 (segment (start 151.8925 81.1765) (end 151.869 81.153) (width 0.6) (layer F.Cu) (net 8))
 (segment (start 155.194 81.1765) (end 151.8925 81.1765) (width 0.6) (layer F.Cu) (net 8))
 (segment (start 158.3685 83.9235) (end 158.392 83.947) (width 0.6) (layer F.Cu) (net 7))
 (segment (start 155.194 83.9235) (end 158.3685 83.9235) (width 0.6) (layer F.Cu) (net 7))
 (segment (start 151.9155 83.9235) (end 151.892 83.947) (width 0.6) (layer F.Cu) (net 7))
 (segment (start 155.194 83.9235) (end 151.9155 83.9235) (width 0.6) (layer F.Cu) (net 7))
 (segment (start 145.1375 79.343) (end 145.106 79.3115) (width 0.4) (layer F.Cu) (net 6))
 (segment (start 145.1375 82.296) (end 145.1375 79.343) (width 0.4) (layer F.Cu) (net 6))
 (segment (start 145.1375 85.78) (end 145.106 85.8115) (width 0.4) (layer F.Cu) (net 6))
 (segment (start 145.1375 82.296) (end 145.1375 85.78) (width 0.4) (layer F.Cu) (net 6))
 (segment (start 136.8025 76.708) (end 136.8025 77.3665) (width 0.6) (layer F.Cu) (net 10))
 (segment (start 141.28949 78.55149) (end 141.986 79.248) (width 0.6) (layer F.Cu) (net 10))
 (segment (start 137.98749 78.55149) (end 141.28949 78.55149) (width 0.6) (layer F.Cu) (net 10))
 (segment (start 136.8025 77.3665) (end 137.98749 78.55149) (width 0.6) (layer F.Cu) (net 10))
 (segment (start 138.451002 85.7485) (end 135.636 85.7485) (width 0.6) (layer F.Cu) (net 1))
 (segment (start 140.014003 87.311501) (end 138.451002 85.7485) (width 0.6) (layer F.Cu) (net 1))
 (segment (start 146.9625 86.175002) (end 145.826001 87.311501) (width 0.6) (layer F.Cu) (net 1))
 (segment (start 146.9625 82.296) (end 146.9625 86.175002) (width 0.6) (layer F.Cu) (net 1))
 (segment (start 141.288499 81.283497) (end 141.288499 87.311501) (width 0.6) (layer F.Cu) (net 1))
 (segment (start 139.356502 79.3515) (end 141.288499 81.283497) (width 0.6) (layer F.Cu) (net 1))
 (segment (start 135.636 79.3515) (end 139.356502 79.3515) (width 0.6) (layer F.Cu) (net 1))
 (segment (start 141.288499 87.311501) (end 140.014003 87.311501) (width 0.6) (layer F.Cu) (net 1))
 (segment (start 145.826001 87.311501) (end 141.288499 87.311501) (width 0.6) (layer F.Cu) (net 1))
 (segment (start 162.4565 78.869998) (end 162.4565 82.55) (width 0.6) (layer F.Cu) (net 1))
 (segment (start 161.375001 77.788499) (end 162.4565 78.869998) (width 0.6) (layer F.Cu) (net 1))
 (segment (start 159.955501 77.788499) (end 161.375001 77.788499) (width 0.6) (layer F.Cu) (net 1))
 (segment (start 158.3925 79.3515) (end 159.955501 77.788499) (width 0.6) (layer F.Cu) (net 1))
 (segment (start 155.194 79.3515) (end 158.3925 79.3515) (width 0.6) (layer F.Cu) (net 1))
 (segment (start 157.913502 85.7485) (end 155.194 85.7485) (width 0.6) (layer F.Cu) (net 1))
 (segment (start 161.375001 87.288501) (end 159.453503 87.288501) (width 0.6) (layer F.Cu) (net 1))
 (segment (start 159.453503 87.288501) (end 157.913502 85.7485) (width 0.6) (layer F.Cu) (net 1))
 (segment (start 162.4565 86.207002) (end 161.375001 87.288501) (width 0.6) (layer F.Cu) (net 1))
 (segment (start 162.4565 82.55) (end 162.4565 86.207002) (width 0.6) (layer F.Cu) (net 1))
 (segment (start 155.194 79.3515) (end 152.2495 79.3515) (width 0.6) (layer F.Cu) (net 1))
 (segment (start 146.9625 77.1125) (end 146.9625 82.296) (width 0.6) (layer F.Cu) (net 1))
 (segment (start 150.0105 77.1125) (end 146.9625 77.1125) (width 0.6) (layer F.Cu) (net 1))
 (segment (start 152.2495 79.3515) (end 150.0105 77.1125) (width 0.6) (layer F.Cu) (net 1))
 (segment (start 145.288 74.168) (end 145.288 76.2) (width 0.6) (layer F.Cu) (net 1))
 (segment (start 146.2005 77.1125) (end 146.9625 77.1125) (width 0.6) (layer F.Cu) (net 1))
 (segment (start 145.288 76.2) (end 146.2005 77.1125) (width 0.6) (layer F.Cu) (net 1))
 (segment (start 142.748 75.946) (end 141.986 76.708) (width 0.6) (layer F.Cu) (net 2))
 (segment (start 142.748 74.168) (end 142.748 75.946) (width 0.6) (layer F.Cu) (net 2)))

